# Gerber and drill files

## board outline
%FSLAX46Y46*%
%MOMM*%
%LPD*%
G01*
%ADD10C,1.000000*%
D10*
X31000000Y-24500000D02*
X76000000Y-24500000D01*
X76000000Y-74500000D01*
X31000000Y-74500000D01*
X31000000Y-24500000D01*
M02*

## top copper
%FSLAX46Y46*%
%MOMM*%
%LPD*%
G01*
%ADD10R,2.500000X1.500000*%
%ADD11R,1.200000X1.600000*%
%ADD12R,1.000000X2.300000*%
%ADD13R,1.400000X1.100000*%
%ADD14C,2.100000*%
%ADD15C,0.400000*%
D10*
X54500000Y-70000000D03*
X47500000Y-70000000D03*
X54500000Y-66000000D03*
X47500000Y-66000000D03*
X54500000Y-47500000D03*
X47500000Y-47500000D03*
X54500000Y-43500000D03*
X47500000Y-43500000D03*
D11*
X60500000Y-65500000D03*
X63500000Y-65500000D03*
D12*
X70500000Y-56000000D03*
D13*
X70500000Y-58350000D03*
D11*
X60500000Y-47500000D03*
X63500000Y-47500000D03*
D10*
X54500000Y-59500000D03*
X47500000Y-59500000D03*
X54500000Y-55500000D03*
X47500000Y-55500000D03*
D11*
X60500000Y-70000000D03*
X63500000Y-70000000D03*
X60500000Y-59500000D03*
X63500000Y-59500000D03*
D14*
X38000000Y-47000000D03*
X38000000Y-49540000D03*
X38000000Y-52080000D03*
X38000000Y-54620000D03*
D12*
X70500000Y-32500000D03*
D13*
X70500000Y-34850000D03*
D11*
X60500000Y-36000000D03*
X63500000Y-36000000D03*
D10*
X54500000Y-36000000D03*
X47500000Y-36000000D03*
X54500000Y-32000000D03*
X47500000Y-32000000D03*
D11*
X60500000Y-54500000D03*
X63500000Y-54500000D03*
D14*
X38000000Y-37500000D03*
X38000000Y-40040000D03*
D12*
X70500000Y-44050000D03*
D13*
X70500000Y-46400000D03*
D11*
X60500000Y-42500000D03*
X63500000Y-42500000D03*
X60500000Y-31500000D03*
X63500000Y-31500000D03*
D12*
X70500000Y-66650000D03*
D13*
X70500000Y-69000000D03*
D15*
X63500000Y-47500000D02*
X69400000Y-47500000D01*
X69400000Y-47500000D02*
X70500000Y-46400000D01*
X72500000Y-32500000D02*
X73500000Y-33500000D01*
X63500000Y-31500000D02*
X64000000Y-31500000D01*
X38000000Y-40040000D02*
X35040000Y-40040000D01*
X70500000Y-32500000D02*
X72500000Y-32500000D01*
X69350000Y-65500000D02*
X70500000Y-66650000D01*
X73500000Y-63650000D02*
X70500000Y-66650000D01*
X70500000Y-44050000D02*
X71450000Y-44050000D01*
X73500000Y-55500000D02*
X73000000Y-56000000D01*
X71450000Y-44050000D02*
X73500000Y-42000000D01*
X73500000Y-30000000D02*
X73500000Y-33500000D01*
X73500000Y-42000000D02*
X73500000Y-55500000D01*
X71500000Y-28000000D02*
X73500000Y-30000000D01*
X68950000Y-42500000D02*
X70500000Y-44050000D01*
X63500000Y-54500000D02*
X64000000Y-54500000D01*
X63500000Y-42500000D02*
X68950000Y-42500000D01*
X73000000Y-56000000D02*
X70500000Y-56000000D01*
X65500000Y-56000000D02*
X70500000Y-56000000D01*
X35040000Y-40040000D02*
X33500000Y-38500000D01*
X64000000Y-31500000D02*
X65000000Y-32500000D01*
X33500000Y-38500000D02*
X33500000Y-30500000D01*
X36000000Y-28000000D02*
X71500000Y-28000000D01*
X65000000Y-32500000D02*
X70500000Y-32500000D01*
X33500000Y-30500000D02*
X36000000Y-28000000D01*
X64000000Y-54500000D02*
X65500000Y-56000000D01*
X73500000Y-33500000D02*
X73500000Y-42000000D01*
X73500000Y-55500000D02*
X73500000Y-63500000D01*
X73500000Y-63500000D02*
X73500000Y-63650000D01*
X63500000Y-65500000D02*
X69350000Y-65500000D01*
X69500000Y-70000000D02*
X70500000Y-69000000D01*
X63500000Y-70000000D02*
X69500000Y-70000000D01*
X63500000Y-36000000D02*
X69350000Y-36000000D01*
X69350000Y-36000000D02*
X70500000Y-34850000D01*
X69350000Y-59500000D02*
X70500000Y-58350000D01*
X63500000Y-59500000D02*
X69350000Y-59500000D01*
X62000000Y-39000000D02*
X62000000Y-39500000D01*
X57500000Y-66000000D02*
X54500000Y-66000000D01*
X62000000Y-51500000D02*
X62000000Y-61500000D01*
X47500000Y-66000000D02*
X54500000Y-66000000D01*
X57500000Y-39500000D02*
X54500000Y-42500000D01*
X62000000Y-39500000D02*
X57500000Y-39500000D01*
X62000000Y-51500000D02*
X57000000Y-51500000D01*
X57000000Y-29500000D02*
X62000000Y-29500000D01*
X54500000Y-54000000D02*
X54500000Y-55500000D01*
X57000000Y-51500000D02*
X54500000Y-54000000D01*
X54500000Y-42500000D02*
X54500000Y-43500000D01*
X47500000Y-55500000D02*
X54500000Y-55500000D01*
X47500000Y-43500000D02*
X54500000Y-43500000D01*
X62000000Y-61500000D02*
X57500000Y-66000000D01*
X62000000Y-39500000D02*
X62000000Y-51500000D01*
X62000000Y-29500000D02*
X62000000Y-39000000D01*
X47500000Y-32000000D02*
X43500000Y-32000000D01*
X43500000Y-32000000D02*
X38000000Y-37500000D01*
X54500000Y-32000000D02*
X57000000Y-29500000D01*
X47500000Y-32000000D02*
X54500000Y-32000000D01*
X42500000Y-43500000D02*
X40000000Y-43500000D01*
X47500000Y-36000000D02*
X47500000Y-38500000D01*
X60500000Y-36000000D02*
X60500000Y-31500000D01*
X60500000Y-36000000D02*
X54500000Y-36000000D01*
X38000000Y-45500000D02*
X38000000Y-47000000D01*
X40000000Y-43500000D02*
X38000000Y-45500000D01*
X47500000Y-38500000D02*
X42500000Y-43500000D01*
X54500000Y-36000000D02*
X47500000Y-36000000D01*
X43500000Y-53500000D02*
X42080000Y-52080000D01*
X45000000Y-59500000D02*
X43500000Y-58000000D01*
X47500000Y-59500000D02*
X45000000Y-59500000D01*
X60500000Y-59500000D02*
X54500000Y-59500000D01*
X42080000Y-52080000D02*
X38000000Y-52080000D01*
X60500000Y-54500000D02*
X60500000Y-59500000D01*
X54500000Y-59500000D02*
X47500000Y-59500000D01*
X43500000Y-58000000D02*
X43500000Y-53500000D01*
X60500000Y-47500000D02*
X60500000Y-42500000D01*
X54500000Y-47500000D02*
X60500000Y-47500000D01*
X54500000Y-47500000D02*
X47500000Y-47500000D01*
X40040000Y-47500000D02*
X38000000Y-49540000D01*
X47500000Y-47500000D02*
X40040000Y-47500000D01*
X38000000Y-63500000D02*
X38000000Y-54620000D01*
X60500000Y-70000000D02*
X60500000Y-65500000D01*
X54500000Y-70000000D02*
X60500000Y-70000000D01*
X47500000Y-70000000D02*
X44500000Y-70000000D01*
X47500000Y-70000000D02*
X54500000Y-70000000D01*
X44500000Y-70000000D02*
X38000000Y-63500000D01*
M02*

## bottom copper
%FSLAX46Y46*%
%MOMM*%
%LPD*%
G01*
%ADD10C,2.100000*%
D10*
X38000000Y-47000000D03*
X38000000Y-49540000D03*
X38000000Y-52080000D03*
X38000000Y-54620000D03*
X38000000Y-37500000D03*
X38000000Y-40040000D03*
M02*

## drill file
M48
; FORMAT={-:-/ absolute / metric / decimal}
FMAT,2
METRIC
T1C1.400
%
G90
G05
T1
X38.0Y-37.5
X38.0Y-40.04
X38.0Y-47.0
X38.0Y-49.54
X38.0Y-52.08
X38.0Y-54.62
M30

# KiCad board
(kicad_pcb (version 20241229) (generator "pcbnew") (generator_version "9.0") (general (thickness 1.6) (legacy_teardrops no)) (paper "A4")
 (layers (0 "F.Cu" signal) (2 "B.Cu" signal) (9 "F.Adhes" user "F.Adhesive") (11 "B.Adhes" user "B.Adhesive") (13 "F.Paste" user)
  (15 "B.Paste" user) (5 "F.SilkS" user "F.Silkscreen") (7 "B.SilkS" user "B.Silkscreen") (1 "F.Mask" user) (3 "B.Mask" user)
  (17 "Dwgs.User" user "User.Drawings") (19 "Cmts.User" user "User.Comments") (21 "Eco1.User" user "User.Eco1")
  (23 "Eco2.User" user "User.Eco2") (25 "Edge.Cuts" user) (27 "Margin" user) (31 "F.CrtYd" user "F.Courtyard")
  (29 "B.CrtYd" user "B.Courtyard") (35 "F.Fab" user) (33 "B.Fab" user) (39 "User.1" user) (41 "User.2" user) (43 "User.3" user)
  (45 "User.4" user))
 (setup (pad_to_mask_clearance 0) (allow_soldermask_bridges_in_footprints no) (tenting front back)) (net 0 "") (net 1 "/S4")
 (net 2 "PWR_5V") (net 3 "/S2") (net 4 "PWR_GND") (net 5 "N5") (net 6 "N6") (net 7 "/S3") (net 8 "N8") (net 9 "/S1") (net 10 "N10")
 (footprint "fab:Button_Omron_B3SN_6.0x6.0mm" (layer "F.Cu") (at 51 68 180)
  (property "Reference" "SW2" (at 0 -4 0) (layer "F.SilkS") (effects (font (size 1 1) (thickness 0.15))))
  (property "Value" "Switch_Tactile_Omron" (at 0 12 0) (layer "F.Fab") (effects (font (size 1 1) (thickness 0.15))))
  (pad "1" smd rect (at -3.5 -2 180) (size 2.5 1.5) (layers "F.Cu" "F.Mask" "F.Paste") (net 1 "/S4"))
  (pad "1" smd rect (at 3.5 -2 180) (size 2.5 1.5) (layers "F.Cu" "F.Mask" "F.Paste") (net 1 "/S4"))
  (pad "2" smd rect (at -3.5 2 180) (size 2.5 1.5) (layers "F.Cu" "F.Mask" "F.Paste") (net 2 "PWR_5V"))
  (pad "2" smd rect (at 3.5 2 180) (size 2.5 1.5) (layers "F.Cu" "F.Mask" "F.Paste") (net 2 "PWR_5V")))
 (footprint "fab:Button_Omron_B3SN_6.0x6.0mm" (layer "F.Cu") (at 51 45.5 180)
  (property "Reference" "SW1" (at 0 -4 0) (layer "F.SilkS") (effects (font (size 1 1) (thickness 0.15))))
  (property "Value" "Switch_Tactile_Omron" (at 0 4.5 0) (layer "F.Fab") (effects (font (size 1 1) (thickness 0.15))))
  (pad "1" smd rect (at -3.5 -2 180) (size 2.5 1.5) (layers "F.Cu" "F.Mask" "F.Paste") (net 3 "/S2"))
  (pad "1" smd rect (at 3.5 -2 180) (size 2.5 1.5) (layers "F.Cu" "F.Mask" "F.Paste") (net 3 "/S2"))
  (pad "2" smd rect (at -3.5 2 180) (size 2.5 1.5) (layers "F.Cu" "F.Mask" "F.Paste") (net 2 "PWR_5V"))
  (pad "2" smd rect (at 3.5 2 180) (size 2.5 1.5) (layers "F.Cu" "F.Mask" "F.Paste") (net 2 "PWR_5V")))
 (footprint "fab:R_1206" (layer "F.Cu") (at 62 65.5)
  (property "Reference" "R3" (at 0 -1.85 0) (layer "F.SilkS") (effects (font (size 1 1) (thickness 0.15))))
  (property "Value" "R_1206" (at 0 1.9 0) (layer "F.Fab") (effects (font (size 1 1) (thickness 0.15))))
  (pad "1" smd rect (at -1.5 0) (size 1.2 1.6) (layers "F.Cu" "F.Mask" "F.Paste") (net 1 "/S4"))
  (pad "2" smd rect (at 1.5 0) (size 1.2 1.6) (layers "F.Cu" "F.Mask" "F.Paste") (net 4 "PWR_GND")))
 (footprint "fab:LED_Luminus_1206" (layer "F.Cu") (at 70.5 56.95 90)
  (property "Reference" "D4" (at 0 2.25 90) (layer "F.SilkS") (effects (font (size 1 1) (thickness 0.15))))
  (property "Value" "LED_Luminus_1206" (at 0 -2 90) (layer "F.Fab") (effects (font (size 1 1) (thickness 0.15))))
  (pad "1" smd rect (at 0.95 0 90) (size 2.3 1) (layers "F.Cu" "F.Mask" "F.Paste") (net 4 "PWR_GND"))
  (pad "2" smd rect (at -1.4 0 90) (size 1.1 1.4) (layers "F.Cu" "F.Mask" "F.Paste") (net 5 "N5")))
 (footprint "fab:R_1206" (layer "F.Cu") (at 62 47.5)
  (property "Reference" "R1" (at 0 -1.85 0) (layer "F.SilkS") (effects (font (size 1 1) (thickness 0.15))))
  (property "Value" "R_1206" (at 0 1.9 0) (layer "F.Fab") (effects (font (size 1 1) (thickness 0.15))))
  (pad "1" smd rect (at -1.5 0) (size 1.2 1.6) (layers "F.Cu" "F.Mask" "F.Paste") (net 3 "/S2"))
  (pad "2" smd rect (at 1.5 0) (size 1.2 1.6) (layers "F.Cu" "F.Mask" "F.Paste") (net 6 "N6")))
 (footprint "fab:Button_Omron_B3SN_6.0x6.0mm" (layer "F.Cu") (at 51 57.5 180)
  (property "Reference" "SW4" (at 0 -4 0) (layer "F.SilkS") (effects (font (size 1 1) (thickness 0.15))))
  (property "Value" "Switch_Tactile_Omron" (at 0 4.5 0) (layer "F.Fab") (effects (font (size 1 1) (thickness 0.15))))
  (pad "1" smd rect (at -3.5 -2 180) (size 2.5 1.5) (layers "F.Cu" "F.Mask" "F.Paste") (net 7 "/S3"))
  (pad "1" smd rect (at 3.5 -2 180) (size 2.5 1.5) (layers "F.Cu" "F.Mask" "F.Paste") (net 7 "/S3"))
  (pad "2" smd rect (at -3.5 2 180) (size 2.5 1.5) (layers "F.Cu" "F.Mask" "F.Paste") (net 2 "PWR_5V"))
  (pad "2" smd rect (at 3.5 2 180) (size 2.5 1.5) (layers "F.Cu" "F.Mask" "F.Paste") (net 2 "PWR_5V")))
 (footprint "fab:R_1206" (layer "F.Cu") (at 62 70)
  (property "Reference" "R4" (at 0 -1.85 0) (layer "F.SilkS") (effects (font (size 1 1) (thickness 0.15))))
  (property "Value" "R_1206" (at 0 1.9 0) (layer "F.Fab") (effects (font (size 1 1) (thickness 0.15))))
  (pad "1" smd rect (at -1.5 0) (size 1.2 1.6) (layers "F.Cu" "F.Mask" "F.Paste") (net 1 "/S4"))
  (pad "2" smd rect (at 1.5 0) (size 1.2 1.6) (layers "F.Cu" "F.Mask" "F.Paste") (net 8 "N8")))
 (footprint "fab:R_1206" (layer "F.Cu") (at 62 59.5)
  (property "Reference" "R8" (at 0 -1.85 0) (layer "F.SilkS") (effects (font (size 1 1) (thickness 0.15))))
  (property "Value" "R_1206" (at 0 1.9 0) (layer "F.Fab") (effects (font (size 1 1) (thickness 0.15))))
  (pad "1" smd rect (at -1.5 0) (size 1.2 1.6) (layers "F.Cu" "F.Mask" "F.Paste") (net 7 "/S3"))
  (pad "2" smd rect (at 1.5 0) (size 1.2 1.6) (layers "F.Cu" "F.Mask" "F.Paste") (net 5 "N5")))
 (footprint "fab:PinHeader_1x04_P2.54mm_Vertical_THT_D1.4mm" (layer "F.Cu") (at 38 47)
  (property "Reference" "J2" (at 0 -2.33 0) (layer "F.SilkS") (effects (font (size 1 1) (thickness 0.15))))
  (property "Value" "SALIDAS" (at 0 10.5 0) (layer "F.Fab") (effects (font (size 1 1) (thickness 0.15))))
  (pad "1" thru_hole circle (at 0 0) (size 2.1 2.1) (drill 1.4) (layers "*.Cu" "*.Mask") (remove_unused_layers no) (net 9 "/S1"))
  (pad "2" thru_hole circle (at 0 2.54) (size 2.1 2.1) (drill 1.4) (layers "*.Cu" "*.Mask") (remove_unused_layers no) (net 3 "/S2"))
  (pad "3" thru_hole circle (at 0 5.08) (size 2.1 2.1) (drill 1.4) (layers "*.Cu" "*.Mask") (remove_unused_layers no) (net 7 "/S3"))
  (pad "4" thru_hole circle (at 0 7.62) (size 2.1 2.1) (drill 1.4) (layers "*.Cu" "*.Mask") (remove_unused_layers no) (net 1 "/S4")))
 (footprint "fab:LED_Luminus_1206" (layer "F.Cu") (at 70.5 33.45 90)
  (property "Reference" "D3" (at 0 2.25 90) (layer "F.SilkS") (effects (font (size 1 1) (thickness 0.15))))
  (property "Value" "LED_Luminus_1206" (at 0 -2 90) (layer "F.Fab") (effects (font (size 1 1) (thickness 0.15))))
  (pad "1" smd rect (at 0.95 0 90) (size 2.3 1) (layers "F.Cu" "F.Mask" "F.Paste") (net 4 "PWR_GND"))
  (pad "2" smd rect (at -1.4 0 90) (size 1.1 1.4) (layers "F.Cu" "F.Mask" "F.Paste") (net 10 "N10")))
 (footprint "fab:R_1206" (layer "F.Cu") (at 62 36)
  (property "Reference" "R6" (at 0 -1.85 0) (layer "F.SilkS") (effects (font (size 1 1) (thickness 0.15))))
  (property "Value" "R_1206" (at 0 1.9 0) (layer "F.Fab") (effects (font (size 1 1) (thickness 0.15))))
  (pad "1" smd rect (at -1.5 0) (size 1.2 1.6) (layers "F.Cu" "F.Mask" "F.Paste") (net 9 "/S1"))
  (pad "2" smd rect (at 1.5 0) (size 1.2 1.6) (layers "F.Cu" "F.Mask" "F.Paste") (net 10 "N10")))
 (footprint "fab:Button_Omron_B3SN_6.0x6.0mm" (layer "F.Cu") (at 51 34 180)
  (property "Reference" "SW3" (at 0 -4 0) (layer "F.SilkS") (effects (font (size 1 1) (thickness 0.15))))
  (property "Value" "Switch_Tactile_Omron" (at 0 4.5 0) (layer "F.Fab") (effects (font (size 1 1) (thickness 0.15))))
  (pad "1" smd rect (at -3.5 -2 180) (size 2.5 1.5) (layers "F.Cu" "F.Mask" "F.Paste") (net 9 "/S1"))
  (pad "1" smd rect (at 3.5 -2 180) (size 2.5 1.5) (layers "F.Cu" "F.Mask" "F.Paste") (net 9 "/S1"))
  (pad "2" smd rect (at -3.5 2 180) (size 2.5 1.5) (layers "F.Cu" "F.Mask" "F.Paste") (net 2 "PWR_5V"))
  (pad "2" smd rect (at 3.5 2 180) (size 2.5 1.5) (layers "F.Cu" "F.Mask" "F.Paste") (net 2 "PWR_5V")))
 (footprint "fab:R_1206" (layer "F.Cu") (at 62 54.5)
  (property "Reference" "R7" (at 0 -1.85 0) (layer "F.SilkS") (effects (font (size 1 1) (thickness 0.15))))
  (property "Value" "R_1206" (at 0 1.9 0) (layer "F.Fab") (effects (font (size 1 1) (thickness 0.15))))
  (pad "1" smd rect (at -1.5 0) (size 1.2 1.6) (layers "F.Cu" "F.Mask" "F.Paste") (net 7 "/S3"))
  (pad "2" smd rect (at 1.5 0) (size 1.2 1.6) (layers "F.Cu" "F.Mask" "F.Paste") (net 4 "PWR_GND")))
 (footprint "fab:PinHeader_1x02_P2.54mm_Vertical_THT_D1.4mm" (layer "F.Cu") (at 38 37.5)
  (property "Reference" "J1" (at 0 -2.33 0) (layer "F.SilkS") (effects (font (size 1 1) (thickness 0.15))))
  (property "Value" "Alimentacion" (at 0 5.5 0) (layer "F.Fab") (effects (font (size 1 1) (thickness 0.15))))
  (pad "1" thru_hole circle (at 0 0) (size 2.1 2.1) (drill 1.4) (layers "*.Cu" "*.Mask") (remove_unused_layers no) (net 2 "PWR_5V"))
  (pad "2" thru_hole circle (at 0 2.54) (size 2.1 2.1) (drill 1.4) (layers "*.Cu" "*.Mask") (remove_unused_layers no) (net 4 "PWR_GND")))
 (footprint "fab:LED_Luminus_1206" (layer "F.Cu") (at 70.5 45 90)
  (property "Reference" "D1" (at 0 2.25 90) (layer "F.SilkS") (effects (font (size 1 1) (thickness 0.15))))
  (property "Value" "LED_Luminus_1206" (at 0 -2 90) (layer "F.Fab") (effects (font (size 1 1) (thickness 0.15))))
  (pad "1" smd rect (at 0.95 0 90) (size 2.3 1) (layers "F.Cu" "F.Mask" "F.Paste") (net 4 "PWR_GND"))
  (pad "2" smd rect (at -1.4 0 90) (size 1.1 1.4) (layers "F.Cu" "F.Mask" "F.Paste") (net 6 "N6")))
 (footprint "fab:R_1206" (layer "F.Cu") (at 62 42.5)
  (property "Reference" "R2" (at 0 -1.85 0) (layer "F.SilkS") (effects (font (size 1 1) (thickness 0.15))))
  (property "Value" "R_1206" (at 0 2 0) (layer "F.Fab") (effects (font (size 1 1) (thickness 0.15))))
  (pad "1" smd rect (at -1.5 0) (size 1.2 1.6) (layers "F.Cu" "F.Mask" "F.Paste") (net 3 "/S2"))
  (pad "2" smd rect (at 1.5 0) (size 1.2 1.6) (layers "F.Cu" "F.Mask" "F.Paste") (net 4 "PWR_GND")))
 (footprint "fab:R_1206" (layer "F.Cu") (at 62 31.5)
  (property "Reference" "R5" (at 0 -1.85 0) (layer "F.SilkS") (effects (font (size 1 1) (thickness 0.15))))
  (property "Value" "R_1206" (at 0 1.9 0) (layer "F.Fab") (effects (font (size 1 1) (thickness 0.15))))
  (pad "1" smd rect (at -1.5 0) (size 1.2 1.6) (layers "F.Cu" "F.Mask" "F.Paste") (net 9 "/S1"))
  (pad "2" smd rect (at 1.5 0) (size 1.2 1.6) (layers "F.Cu" "F.Mask" "F.Paste") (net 4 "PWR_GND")))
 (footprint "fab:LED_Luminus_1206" (layer "F.Cu") (at 70.5 67.6 90)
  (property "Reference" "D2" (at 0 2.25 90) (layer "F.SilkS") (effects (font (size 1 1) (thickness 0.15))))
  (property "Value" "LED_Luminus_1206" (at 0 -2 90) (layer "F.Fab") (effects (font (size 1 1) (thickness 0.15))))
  (pad "1" smd rect (at 0.95 0 90) (size 2.3 1) (layers "F.Cu" "F.Mask" "F.Paste") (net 4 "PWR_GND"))
  (pad "2" smd rect (at -1.4 0 90) (size 1.1 1.4) (layers "F.Cu" "F.Mask" "F.Paste") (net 8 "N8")))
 (gr_rect (start 31 24.5) (end 76 74.5) (stroke (width 1) (type solid)) (fill no) (layer "Edge.Cuts"))
 (segment (start 63.5 47.5) (end 69.4 47.5) (width 0.4) (layer "F.Cu") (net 6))
 (segment (start 69.4 47.5) (end 70.5 46.4) (width 0.4) (layer "F.Cu") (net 6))
 (segment (start 72.5 32.5) (end 73.5 33.5) (width 0.4) (layer "F.Cu") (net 4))
 (segment (start 63.5 31.5) (end 64 31.5) (width 0.4) (layer "F.Cu") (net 4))
 (segment (start 38 40.04) (end 35.04 40.04) (width 0.4) (layer "F.Cu") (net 4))
 (segment (start 70.5 32.5) (end 72.5 32.5) (width 0.4) (layer "F.Cu") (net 4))
 (segment (start 69.35 65.5) (end 70.5 66.65) (width 0.4) (layer "F.Cu") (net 4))
 (segment (start 73.5 63.65) (end 70.5 66.65) (width 0.4) (layer "F.Cu") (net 4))
 (segment (start 70.5 44.05) (end 71.45 44.05) (width 0.4) (layer "F.Cu") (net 4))
 (segment (start 73.5 55.5) (end 73 56) (width 0.4) (layer "F.Cu") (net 4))
 (segment (start 71.45 44.05) (end 73.5 42) (width 0.4) (layer "F.Cu") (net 4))
 (segment (start 73.5 30) (end 73.5 33.5) (width 0.4) (layer "F.Cu") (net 4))
 (segment (start 73.5 42) (end 73.5 55.5) (width 0.4) (layer "F.Cu") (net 4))
 (segment (start 71.5 28) (end 73.5 30) (width 0.4) (layer "F.Cu") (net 4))
 (segment (start 68.95 42.5) (end 70.5 44.05) (width 0.4) (layer "F.Cu") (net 4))
 (segment (start 63.5 54.5) (end 64 54.5) (width 0.4) (layer "F.Cu") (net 4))
 (segment (start 63.5 42.5) (end 68.95 42.5) (width 0.4) (layer "F.Cu") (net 4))
 (segment (start 73 56) (end 70.5 56) (width 0.4) (layer "F.Cu") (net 4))
 (segment (start 65.5 56) (end 70.5 56) (width 0.4) (layer "F.Cu") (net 4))
 (segment (start 35.04 40.04) (end 33.5 38.5) (width 0.4) (layer "F.Cu") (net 4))
 (segment (start 64 31.5) (end 65 32.5) (width 0.4) (layer "F.Cu") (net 4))
 (segment (start 33.5 38.5) (end 33.5 30.5) (width 0.4) (layer "F.Cu") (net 4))
 (segment (start 36 28) (end 71.5 28) (width 0.4) (layer "F.Cu") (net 4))
 (segment (start 65 32.5) (end 70.5 32.5) (width 0.4) (layer "F.Cu") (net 4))
 (segment (start 33.5 30.5) (end 36 28) (width 0.4) (layer "F.Cu") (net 4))
 (segment (start 64 54.5) (end 65.5 56) (width 0.4) (layer "F.Cu") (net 4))
 (segment (start 73.5 33.5) (end 73.5 42) (width 0.4) (layer "F.Cu") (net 4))
 (segment (start 73.5 55.5) (end 73.5 63.5) (width 0.4) (layer "F.Cu") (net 4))
 (segment (start 73.5 63.5) (end 73.5 63.65) (width 0.4) (layer "F.Cu") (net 4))
 (segment (start 63.5 65.5) (end 69.35 65.5) (width 0.4) (layer "F.Cu") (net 4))
 (segment (start 69.5 70) (end 70.5 69) (width 0.4) (layer "F.Cu") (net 8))
 (segment (start 63.5 70) (end 69.5 70) (width 0.4) (layer "F.Cu") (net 8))
 (segment (start 63.5 36) (end 69.35 36) (width 0.4) (layer "F.Cu") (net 10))
 (segment (start 69.35 36) (end 70.5 34.85) (width 0.4) (layer "F.Cu") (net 10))
 (segment (start 69.35 59.5) (end 70.5 58.35) (width 0.4) (layer "F.Cu") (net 5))
 (segment (start 63.5 59.5) (end 69.35 59.5) (width 0.4) (layer "F.Cu") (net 5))
 (segment (start 62 39) (end 62 39.5) (width 0.4) (layer "F.Cu") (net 2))
 (segment (start 57.5 66) (end 54.5 66) (width 0.4) (layer "F.Cu") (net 2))
 (segment (start 62 51.5) (end 62 61.5) (width 0.4) (layer "F.Cu") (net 2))
 (segment (start 47.5 66) (end 54.5 66) (width 0.4) (layer "F.Cu") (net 2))
 (segment (start 57.5 39.5) (end 54.5 42.5) (width 0.4) (layer "F.Cu") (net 2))
 (segment (start 62 39.5) (end 57.5 39.5) (width 0.4) (layer "F.Cu") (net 2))
 (segment (start 62 51.5) (end 57 51.5) (width 0.4) (layer "F.Cu") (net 2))
 (segment (start 57 29.5) (end 62 29.5) (width 0.4) (layer "F.Cu") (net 2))
 (segment (start 54.5 54) (end 54.5 55.5) (width 0.4) (layer "F.Cu") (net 2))
 (segment (start 57 51.5) (end 54.5 54) (width 0.4) (layer "F.Cu") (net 2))
 (segment (start 54.5 42.5) (end 54.5 43.5) (width 0.4) (layer "F.Cu") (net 2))
 (segment (start 47.5 55.5) (end 54.5 55.5) (width 0.4) (layer "F.Cu") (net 2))
 (segment (start 47.5 43.5) (end 54.5 43.5) (width 0.4) (layer "F.Cu") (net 2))
 (segment (start 62 61.5) (end 57.5 66) (width 0.4) (layer "F.Cu") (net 2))
 (segment (start 62 39.5) (end 62 51.5) (width 0.4) (layer "F.Cu") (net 2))
 (segment (start 62 29.5) (end 62 39) (width 0.4) (layer "F.Cu") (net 2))
 (segment (start 47.5 32) (end 43.5 32) (width 0.4) (layer "F.Cu") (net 2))
 (segment (start 43.5 32) (end 38 37.5) (width 0.4) (layer "F.Cu") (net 2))
 (segment (start 54.5 32) (end 57 29.5) (width 0.4) (layer "F.Cu") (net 2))
 (segment (start 47.5 32) (end 54.5 32) (width 0.4) (layer "F.Cu") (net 2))
 (segment (start 42.5 43.5) (end 40 43.5) (width 0.4) (layer "F.Cu") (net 9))
 (segment (start 47.5 36) (end 47.5 38.5) (width 0.4) (layer "F.Cu") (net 9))
 (segment (start 60.5 36) (end 60.5 31.5) (width 0.4) (layer "F.Cu") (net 9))
 (segment (start 60.5 36) (end 54.5 36) (width 0.4) (layer "F.Cu") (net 9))
 (segment (start 38 45.5) (end 38 47) (width 0.4) (layer "F.Cu") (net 9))
 (segment (start 40 43.5) (end 38 45.5) (width 0.4) (layer "F.Cu") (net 9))
 (segment (start 47.5 38.5) (end 42.5 43.5) (width 0.4) (layer "F.Cu") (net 9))
 (segment (start 54.5 36) (end 47.5 36) (width 0.4) (layer "F.Cu") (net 9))
 (segment (start 43.5 53.5) (end 42.08 52.08) (width 0.4) (layer "F.Cu") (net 7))
 (segment (start 45 59.5) (end 43.5 58) (width 0.4) (layer "F.Cu") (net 7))
 (segment (start 47.5 59.5) (end 45 59.5) (width 0.4) (layer "F.Cu") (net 7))
 (segment (start 60.5 59.5) (end 54.5 59.5) (width 0.4) (layer "F.Cu") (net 7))
 (segment (start 42.08 52.08) (end 38 52.08) (width 0.4) (layer "F.Cu") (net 7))
 (segment (start 60.5 54.5) (end 60.5 59.5) (width 0.4) (layer "F.Cu") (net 7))
 (segment (start 54.5 59.5) (end 47.5 59.5) (width 0.4) (layer "F.Cu") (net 7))
 (segment (start 43.5 58) (end 43.5 53.5) (width 0.4) (layer "F.Cu") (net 7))
 (segment (start 60.5 47.5) (end 60.5 42.5) (width 0.4) (layer "F.Cu") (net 3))
 (segment (start 54.5 47.5) (end 60.5 47.5) (width 0.4) (layer "F.Cu") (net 3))
 (segment (start 54.5 47.5) (end 47.5 47.5) (width 0.4) (layer "F.Cu") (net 3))
 (segment (start 40.04 47.5) (end 38 49.54) (width 0.4) (layer "F.Cu") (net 3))
 (segment (start 47.5 47.5) (end 40.04 47.5) (width 0.4) (layer "F.Cu") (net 3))
 (segment (start 38 63.5) (end 38 54.62) (width 0.4) (layer "F.Cu") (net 1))
 (segment (start 60.5 70) (end 60.5 65.5) (width 0.4) (layer "F.Cu") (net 1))
 (segment (start 54.5 70) (end 60.5 70) (width 0.4) (layer "F.Cu") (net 1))
 (segment (start 47.5 70) (end 44.5 70) (width 0.4) (layer "F.Cu") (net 1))
 (segment (start 47.5 70) (end 54.5 70) (width 0.4) (layer "F.Cu") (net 1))
 (segment (start 44.5 70) (end 38 63.5) (width 0.4) (layer "F.Cu") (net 1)))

